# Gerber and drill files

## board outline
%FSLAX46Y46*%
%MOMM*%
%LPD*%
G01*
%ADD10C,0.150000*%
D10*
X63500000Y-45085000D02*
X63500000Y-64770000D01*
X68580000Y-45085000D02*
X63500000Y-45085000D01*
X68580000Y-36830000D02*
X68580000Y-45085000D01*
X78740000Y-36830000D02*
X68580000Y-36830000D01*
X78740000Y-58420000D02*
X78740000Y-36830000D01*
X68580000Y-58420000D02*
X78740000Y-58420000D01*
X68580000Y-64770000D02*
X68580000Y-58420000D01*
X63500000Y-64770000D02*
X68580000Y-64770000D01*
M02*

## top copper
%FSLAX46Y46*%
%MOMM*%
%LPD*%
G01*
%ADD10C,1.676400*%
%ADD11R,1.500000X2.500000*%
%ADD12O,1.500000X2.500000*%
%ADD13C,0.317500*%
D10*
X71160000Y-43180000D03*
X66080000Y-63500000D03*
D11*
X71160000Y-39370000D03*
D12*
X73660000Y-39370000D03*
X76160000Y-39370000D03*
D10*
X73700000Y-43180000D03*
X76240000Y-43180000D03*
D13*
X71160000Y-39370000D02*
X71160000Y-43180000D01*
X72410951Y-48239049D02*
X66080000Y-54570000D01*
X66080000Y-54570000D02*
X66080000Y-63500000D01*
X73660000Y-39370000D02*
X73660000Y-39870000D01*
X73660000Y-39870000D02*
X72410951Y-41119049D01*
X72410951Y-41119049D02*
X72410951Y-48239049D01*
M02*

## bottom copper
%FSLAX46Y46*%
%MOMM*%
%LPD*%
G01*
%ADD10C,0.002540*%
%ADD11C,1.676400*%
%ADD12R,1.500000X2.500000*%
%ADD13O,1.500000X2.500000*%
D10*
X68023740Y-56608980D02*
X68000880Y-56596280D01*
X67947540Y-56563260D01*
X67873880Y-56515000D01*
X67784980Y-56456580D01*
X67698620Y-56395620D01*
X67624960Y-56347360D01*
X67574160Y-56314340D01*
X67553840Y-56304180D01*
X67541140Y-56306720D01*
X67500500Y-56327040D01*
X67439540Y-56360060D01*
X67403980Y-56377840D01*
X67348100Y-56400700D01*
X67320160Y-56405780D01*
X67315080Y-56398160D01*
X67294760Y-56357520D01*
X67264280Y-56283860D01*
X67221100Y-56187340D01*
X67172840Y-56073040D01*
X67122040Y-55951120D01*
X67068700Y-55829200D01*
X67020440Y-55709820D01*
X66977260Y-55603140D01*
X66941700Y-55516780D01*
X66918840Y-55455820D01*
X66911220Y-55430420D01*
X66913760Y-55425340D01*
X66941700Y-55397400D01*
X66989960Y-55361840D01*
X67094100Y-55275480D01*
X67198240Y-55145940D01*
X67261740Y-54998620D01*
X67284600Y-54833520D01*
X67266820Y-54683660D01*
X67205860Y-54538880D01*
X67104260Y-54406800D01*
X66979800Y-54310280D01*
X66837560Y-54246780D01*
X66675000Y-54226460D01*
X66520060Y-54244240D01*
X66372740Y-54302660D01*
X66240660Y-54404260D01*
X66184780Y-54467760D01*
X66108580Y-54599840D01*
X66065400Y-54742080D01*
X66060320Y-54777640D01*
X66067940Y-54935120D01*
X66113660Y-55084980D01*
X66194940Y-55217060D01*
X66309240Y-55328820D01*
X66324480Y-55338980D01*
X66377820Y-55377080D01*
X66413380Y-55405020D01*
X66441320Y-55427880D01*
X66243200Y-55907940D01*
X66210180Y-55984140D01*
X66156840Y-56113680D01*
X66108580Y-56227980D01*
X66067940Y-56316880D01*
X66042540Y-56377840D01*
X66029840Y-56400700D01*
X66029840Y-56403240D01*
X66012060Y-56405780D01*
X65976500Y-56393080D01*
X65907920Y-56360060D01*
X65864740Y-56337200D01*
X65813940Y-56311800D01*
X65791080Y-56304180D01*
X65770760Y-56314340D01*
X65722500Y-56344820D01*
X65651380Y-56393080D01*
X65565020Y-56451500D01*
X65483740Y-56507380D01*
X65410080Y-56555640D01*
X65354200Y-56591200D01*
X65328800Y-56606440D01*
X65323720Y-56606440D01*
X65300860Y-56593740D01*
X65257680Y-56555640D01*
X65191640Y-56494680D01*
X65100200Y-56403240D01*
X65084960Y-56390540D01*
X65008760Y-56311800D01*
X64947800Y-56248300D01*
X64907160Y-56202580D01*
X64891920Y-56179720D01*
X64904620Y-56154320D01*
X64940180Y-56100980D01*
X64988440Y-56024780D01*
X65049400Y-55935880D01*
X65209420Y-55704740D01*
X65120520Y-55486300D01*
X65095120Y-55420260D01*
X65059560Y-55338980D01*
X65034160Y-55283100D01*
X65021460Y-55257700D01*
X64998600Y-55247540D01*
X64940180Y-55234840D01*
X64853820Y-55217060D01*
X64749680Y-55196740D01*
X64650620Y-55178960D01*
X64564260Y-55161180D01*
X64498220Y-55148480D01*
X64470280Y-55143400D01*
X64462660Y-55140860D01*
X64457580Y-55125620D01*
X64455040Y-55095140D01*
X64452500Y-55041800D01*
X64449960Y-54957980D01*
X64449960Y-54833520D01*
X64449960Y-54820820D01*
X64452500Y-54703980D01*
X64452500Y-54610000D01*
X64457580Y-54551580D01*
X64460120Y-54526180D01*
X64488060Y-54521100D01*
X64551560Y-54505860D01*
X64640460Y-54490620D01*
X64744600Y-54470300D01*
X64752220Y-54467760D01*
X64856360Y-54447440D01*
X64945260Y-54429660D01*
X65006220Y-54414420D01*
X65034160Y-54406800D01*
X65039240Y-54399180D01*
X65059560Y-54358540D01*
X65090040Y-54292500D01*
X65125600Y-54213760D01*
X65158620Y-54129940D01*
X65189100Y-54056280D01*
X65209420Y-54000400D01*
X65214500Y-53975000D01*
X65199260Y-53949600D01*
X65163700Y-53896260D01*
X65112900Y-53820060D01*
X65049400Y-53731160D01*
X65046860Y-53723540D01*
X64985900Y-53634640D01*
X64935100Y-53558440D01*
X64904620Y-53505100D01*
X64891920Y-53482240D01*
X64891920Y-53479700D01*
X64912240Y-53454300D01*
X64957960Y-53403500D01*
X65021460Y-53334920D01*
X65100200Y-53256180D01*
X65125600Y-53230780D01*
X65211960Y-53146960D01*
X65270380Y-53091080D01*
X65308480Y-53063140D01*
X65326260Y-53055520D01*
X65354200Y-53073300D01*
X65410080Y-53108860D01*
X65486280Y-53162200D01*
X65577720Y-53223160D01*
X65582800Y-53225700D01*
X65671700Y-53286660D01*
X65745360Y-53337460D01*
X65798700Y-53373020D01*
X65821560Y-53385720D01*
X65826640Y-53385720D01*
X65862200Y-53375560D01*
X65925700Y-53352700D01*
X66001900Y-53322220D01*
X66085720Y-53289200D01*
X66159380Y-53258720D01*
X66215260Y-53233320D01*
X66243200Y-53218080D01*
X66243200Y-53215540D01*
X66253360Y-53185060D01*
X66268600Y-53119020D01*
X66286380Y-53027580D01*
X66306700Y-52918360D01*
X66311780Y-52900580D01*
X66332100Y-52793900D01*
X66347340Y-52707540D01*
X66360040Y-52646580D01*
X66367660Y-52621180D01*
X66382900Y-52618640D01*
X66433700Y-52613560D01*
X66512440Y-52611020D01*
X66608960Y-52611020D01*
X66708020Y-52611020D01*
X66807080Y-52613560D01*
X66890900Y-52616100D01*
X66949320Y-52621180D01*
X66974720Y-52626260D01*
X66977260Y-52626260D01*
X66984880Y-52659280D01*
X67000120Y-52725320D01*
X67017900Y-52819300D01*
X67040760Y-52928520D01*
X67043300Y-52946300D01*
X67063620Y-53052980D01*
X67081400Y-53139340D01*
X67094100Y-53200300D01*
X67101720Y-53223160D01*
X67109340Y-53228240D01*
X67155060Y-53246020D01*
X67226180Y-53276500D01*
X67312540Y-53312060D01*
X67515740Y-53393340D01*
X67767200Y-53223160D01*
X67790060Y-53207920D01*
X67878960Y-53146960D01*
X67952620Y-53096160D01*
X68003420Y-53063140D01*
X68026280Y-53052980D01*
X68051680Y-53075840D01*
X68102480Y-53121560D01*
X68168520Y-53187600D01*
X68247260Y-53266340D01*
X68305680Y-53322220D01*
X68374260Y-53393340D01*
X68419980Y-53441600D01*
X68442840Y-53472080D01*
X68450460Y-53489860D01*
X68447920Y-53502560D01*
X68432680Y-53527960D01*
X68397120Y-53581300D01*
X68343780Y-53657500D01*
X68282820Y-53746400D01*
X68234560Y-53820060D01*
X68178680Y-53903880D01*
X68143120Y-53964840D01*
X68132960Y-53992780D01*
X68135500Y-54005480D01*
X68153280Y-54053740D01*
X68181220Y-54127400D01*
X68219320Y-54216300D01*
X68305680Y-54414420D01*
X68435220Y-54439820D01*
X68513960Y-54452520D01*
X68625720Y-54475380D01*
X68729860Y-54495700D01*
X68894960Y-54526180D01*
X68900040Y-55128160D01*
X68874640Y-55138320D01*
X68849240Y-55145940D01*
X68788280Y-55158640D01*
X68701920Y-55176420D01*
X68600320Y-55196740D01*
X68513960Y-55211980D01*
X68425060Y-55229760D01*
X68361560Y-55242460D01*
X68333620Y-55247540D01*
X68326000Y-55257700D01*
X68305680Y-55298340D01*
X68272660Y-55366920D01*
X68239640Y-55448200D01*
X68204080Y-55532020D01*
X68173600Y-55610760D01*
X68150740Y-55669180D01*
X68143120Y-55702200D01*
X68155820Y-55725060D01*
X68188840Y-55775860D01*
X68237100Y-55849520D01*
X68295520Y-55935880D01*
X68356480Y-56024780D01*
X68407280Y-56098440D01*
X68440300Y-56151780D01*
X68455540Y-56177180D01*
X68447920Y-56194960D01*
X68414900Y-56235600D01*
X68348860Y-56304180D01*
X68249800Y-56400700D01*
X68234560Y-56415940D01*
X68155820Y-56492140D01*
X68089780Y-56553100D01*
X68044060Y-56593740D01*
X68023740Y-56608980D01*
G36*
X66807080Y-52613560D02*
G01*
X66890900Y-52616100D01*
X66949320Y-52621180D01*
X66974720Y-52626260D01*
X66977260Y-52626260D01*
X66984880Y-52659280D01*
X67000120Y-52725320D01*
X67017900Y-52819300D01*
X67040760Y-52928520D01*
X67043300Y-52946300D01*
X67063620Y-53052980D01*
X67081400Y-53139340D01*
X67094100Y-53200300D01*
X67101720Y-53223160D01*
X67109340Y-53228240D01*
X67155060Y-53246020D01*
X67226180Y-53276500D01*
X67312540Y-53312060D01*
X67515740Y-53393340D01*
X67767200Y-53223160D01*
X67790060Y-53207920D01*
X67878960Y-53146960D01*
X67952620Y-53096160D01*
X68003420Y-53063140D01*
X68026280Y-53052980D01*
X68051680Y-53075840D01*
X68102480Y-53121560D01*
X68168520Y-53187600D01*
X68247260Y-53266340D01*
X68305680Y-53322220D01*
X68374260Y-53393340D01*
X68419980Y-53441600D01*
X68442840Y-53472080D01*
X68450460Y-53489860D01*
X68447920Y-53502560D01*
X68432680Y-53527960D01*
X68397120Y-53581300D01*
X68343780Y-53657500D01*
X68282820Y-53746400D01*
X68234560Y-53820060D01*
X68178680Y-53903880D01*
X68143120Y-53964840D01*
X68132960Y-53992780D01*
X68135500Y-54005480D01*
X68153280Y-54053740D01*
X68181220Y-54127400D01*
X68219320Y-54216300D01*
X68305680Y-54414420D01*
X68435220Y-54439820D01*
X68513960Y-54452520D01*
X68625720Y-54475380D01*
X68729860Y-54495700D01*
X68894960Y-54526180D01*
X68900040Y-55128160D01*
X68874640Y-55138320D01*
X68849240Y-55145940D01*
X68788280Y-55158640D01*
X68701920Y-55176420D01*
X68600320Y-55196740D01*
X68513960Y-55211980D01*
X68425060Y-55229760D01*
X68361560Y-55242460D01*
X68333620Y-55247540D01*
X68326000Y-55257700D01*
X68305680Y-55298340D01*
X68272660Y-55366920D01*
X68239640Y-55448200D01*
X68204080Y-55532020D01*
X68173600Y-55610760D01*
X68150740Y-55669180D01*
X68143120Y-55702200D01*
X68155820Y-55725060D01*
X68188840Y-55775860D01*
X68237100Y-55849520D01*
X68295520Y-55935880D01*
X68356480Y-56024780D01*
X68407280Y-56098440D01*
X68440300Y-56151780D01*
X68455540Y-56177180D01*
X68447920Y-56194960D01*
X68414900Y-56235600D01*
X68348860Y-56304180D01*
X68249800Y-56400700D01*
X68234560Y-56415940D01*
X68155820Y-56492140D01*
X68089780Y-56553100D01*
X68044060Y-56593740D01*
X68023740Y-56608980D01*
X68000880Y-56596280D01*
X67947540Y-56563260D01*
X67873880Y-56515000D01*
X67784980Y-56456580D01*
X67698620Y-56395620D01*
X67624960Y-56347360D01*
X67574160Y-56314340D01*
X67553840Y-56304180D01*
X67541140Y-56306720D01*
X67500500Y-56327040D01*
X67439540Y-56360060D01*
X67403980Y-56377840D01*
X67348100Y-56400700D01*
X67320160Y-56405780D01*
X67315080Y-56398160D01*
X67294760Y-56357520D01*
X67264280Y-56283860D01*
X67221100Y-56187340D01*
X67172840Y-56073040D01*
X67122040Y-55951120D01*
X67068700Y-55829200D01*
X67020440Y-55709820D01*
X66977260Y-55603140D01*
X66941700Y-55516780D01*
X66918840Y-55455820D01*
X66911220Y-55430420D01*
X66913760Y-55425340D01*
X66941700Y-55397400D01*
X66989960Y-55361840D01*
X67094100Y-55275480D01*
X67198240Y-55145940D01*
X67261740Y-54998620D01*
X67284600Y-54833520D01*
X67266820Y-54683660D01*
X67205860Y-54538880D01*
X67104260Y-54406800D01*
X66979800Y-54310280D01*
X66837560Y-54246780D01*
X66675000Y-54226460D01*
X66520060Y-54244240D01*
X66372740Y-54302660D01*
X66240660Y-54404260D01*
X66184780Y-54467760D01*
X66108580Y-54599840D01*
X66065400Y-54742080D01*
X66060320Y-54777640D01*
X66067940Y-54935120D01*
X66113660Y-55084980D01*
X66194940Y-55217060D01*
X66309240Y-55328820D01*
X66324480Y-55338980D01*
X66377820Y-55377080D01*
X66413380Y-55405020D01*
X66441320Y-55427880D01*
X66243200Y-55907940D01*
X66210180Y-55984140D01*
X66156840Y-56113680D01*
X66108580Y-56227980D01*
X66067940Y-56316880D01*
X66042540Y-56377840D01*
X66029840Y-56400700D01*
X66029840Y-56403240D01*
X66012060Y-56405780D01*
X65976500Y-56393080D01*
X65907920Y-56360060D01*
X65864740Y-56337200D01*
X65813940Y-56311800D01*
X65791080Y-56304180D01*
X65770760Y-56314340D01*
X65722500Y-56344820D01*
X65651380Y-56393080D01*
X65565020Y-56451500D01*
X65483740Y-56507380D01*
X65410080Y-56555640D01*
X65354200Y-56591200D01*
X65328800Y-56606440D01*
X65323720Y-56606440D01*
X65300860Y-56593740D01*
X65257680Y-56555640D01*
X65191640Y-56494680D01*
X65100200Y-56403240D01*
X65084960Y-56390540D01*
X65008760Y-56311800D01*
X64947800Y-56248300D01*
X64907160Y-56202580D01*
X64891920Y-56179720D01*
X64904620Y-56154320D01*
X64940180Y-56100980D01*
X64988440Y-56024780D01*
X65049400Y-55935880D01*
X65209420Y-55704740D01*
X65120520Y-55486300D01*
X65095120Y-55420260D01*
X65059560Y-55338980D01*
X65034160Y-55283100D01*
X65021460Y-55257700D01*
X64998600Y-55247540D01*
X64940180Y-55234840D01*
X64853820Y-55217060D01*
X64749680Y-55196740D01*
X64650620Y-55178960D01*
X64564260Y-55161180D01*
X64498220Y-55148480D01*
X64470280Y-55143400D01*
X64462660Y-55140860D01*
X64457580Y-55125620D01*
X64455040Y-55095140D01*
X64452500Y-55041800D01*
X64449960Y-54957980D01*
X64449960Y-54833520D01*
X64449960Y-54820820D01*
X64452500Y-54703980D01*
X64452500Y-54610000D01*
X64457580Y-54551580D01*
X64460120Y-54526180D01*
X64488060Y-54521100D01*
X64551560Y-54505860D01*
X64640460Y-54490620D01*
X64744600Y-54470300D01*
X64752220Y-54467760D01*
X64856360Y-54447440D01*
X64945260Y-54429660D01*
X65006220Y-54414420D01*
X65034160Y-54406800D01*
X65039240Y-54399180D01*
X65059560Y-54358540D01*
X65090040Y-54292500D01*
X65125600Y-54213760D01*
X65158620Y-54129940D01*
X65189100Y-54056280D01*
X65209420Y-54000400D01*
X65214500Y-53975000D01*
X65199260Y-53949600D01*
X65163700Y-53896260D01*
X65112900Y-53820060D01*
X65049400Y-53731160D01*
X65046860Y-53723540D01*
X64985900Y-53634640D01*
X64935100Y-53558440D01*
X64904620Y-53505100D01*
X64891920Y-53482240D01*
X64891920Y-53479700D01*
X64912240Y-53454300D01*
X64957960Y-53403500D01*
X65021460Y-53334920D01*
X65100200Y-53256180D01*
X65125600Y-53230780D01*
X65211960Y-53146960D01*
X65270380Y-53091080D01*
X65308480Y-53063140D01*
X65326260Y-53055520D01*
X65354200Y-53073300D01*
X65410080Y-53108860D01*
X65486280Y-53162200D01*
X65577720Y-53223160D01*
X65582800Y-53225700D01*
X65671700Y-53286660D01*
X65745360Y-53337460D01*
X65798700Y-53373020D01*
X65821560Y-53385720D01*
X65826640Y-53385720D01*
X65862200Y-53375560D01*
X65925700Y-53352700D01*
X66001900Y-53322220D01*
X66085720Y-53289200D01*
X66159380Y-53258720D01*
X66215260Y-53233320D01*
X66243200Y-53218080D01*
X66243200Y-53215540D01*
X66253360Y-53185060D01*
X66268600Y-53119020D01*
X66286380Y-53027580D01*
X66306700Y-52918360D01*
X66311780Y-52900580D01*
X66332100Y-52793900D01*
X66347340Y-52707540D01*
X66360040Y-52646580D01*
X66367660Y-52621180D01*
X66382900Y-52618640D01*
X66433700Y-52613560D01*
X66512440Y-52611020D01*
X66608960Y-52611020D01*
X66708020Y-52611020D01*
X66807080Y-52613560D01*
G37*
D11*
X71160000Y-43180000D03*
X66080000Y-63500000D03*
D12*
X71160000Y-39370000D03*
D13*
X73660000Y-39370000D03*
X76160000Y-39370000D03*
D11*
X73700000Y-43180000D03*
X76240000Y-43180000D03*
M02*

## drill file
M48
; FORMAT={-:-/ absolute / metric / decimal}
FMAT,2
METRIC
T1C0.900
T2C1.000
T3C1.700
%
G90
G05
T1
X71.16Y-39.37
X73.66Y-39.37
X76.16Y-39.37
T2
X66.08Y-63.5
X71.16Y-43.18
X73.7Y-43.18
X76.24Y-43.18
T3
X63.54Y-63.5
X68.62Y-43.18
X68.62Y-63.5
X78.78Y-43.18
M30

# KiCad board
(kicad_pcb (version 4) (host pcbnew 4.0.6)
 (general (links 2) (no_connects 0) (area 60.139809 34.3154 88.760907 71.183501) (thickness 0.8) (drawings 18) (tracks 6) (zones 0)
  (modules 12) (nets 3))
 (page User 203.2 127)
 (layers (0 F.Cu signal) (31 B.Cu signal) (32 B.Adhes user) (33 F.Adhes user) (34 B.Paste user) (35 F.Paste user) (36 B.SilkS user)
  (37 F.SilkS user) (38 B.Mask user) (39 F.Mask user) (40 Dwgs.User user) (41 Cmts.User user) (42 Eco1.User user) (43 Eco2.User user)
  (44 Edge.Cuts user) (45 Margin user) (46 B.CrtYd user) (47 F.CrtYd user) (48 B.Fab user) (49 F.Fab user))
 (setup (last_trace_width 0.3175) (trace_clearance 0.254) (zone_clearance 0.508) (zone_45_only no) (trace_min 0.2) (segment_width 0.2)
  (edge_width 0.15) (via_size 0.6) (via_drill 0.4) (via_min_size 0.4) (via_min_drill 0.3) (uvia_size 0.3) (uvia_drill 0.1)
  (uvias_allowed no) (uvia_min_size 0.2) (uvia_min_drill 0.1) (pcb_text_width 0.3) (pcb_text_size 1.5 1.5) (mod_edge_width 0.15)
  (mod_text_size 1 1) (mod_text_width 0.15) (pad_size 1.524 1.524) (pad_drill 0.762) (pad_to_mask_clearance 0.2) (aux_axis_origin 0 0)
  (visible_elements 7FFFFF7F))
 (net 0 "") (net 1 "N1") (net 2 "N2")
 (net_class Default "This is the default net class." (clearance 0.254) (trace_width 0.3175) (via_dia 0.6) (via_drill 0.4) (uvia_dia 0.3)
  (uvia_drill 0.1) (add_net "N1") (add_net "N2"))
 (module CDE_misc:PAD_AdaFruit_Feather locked (layer F.Cu) (at 71.12 43.18)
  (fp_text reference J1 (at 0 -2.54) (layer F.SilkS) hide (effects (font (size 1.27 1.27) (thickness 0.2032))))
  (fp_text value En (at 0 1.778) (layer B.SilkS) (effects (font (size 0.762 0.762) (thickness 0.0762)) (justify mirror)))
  (pad 1 thru_hole circle (at 0.04 0) (size 1.6764 1.6764) (drill 1) (layers *.Cu *.Mask) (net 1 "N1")))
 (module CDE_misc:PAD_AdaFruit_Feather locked (layer F.Cu) (at 66.04 63.5)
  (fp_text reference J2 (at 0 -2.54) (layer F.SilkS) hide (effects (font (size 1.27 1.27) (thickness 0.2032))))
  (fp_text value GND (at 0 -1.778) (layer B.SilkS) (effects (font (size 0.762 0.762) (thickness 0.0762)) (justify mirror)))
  (pad 1 thru_hole circle (at 0.04 0) (size 1.6764 1.6764) (drill 1) (layers *.Cu *.Mask) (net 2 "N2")))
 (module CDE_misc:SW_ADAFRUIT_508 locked (layer F.Cu) (at 71.12 39.37)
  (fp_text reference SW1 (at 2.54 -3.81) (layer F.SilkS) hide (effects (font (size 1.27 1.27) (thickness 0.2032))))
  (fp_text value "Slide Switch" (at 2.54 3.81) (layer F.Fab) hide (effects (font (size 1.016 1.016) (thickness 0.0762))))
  (pad 1 thru_hole rect (at 0.04 0) (size 1.5 2.5) (drill 0.9) (layers *.Cu *.Mask) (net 1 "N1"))
  (pad 2 thru_hole oval (at 2.54 0) (size 1.5 2.5) (drill 0.9) (layers *.Cu *.Mask) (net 2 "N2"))
  (pad 3 thru_hole oval (at 5.04 0) (size 1.5 2.5) (drill 0.9) (layers *.Cu *.Mask)))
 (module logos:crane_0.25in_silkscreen (layer B.Cu) (at 73.66 53.975 180)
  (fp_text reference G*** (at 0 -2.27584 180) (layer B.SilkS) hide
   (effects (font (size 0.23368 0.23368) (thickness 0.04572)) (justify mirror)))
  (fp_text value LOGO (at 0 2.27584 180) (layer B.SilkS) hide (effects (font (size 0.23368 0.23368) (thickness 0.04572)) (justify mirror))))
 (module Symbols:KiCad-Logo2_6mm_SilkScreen (layer F.Cu) (at 71.12 54.61)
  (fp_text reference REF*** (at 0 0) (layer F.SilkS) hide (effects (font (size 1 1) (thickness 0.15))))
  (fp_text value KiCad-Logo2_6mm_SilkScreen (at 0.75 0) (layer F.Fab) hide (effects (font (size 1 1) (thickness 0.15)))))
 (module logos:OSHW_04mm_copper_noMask (layer B.Cu) (at 66.675 54.61 180)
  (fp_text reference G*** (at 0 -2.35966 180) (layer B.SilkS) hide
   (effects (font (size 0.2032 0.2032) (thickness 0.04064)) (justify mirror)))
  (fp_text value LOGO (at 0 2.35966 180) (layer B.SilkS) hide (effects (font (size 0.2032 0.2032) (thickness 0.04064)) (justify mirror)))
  (fp_poly
   (pts (xy -1.34874 -1.99898) (xy -1.32588 -1.98628) (xy -1.27254 -1.95326) (xy -1.19888 -1.905) (xy -1.10998 -1.84658)
    (xy -1.02362 -1.78562) (xy -0.94996 -1.73736) (xy -0.89916 -1.70434) (xy -0.87884 -1.69418) (xy -0.86614 -1.69672) (xy -0.8255 -1.71704)
    (xy -0.76454 -1.75006) (xy -0.72898 -1.76784) (xy -0.6731 -1.7907) (xy -0.64516 -1.79578) (xy -0.64008 -1.78816) (xy -0.61976 -1.74752)
    (xy -0.58928 -1.67386) (xy -0.5461 -1.57734) (xy -0.49784 -1.46304) (xy -0.44704 -1.34112) (xy -0.3937 -1.2192) (xy -0.34544 -1.09982)
    (xy -0.30226 -0.99314) (xy -0.2667 -0.90678) (xy -0.24384 -0.84582) (xy -0.23622 -0.82042) (xy -0.23876 -0.81534) (xy -0.2667 -0.7874)
    (xy -0.31496 -0.75184) (xy -0.4191 -0.66548) (xy -0.52324 -0.53594) (xy -0.58674 -0.38862) (xy -0.6096 -0.22352) (xy -0.59182 -0.07366)
    (xy -0.53086 0.07112) (xy -0.42926 0.2032) (xy -0.3048 0.29972) (xy -0.16256 0.36322) (xy 0 0.38354) (xy 0.15494 0.36576)
    (xy 0.30226 0.30734) (xy 0.43434 0.20574) (xy 0.49022 0.14224) (xy 0.56642 0.01016) (xy 0.6096 -0.13208) (xy 0.61468 -0.16764)
    (xy 0.60706 -0.32512) (xy 0.56134 -0.47498) (xy 0.48006 -0.60706) (xy 0.36576 -0.71882) (xy 0.35052 -0.72898) (xy 0.29718 -0.76708)
    (xy 0.26162 -0.79502) (xy 0.23368 -0.81788) (xy 0.4318 -1.29794) (xy 0.46482 -1.37414) (xy 0.51816 -1.50368) (xy 0.56642 -1.61798)
    (xy 0.60706 -1.70688) (xy 0.63246 -1.76784) (xy 0.64516 -1.7907) (xy 0.64516 -1.79324) (xy 0.66294 -1.79578) (xy 0.6985 -1.78308)
    (xy 0.76708 -1.75006) (xy 0.81026 -1.7272) (xy 0.86106 -1.7018) (xy 0.88392 -1.69418) (xy 0.90424 -1.70434) (xy 0.9525 -1.73482)
    (xy 1.02362 -1.78308) (xy 1.10998 -1.8415) (xy 1.19126 -1.89738) (xy 1.26492 -1.94564) (xy 1.3208 -1.9812) (xy 1.3462 -1.99644)
    (xy 1.35128 -1.99644) (xy 1.37414 -1.98374) (xy 1.41732 -1.94564) (xy 1.48336 -1.88468) (xy 1.5748 -1.79324) (xy 1.59004 -1.78054)
    (xy 1.66624 -1.7018) (xy 1.7272 -1.6383) (xy 1.76784 -1.59258) (xy 1.78308 -1.56972) (xy 1.78308 -1.56972) (xy 1.77038 -1.54432)
    (xy 1.73482 -1.49098) (xy 1.68656 -1.41478) (xy 1.6256 -1.32588) (xy 1.46558 -1.09474) (xy 1.55448 -0.8763) (xy 1.57988 -0.81026)
    (xy 1.61544 -0.72898) (xy 1.64084 -0.6731) (xy 1.65354 -0.6477) (xy 1.6764 -0.63754) (xy 1.73482 -0.62484) (xy 1.82118 -0.60706)
    (xy 1.92532 -0.58674) (xy 2.02438 -0.56896) (xy 2.11074 -0.55118) (xy 2.17678 -0.53848) (xy 2.20472 -0.5334) (xy 2.21234 -0.53086)
    (xy 2.21742 -0.51562) (xy 2.21996 -0.48514) (xy 2.2225 -0.4318) (xy 2.22504 -0.34798) (xy 2.22504 -0.22352) (xy 2.22504 -0.21082)
    (xy 2.2225 -0.09398) (xy 2.2225 0) (xy 2.21742 0.05842) (xy 2.21488 0.08382) (xy 2.21488 0.08382) (xy 2.18694 0.0889)
    (xy 2.12344 0.10414) (xy 2.03454 0.11938) (xy 1.9304 0.1397) (xy 1.92278 0.14224) (xy 1.81864 0.16256) (xy 1.72974 0.18034)
    (xy 1.66878 0.19558) (xy 1.64084 0.2032) (xy 1.63576 0.21082) (xy 1.61544 0.25146) (xy 1.58496 0.3175) (xy 1.5494 0.39624)
    (xy 1.51638 0.48006) (xy 1.4859 0.55372) (xy 1.46558 0.6096) (xy 1.4605 0.635) (xy 1.4605 0.635) (xy 1.47574 0.6604) (xy 1.5113 0.71374)
    (xy 1.5621 0.78994) (xy 1.6256 0.87884) (xy 1.62814 0.88646) (xy 1.6891 0.97536) (xy 1.7399 1.05156) (xy 1.77038 1.1049)
    (xy 1.78308 1.12776) (xy 1.78308 1.1303) (xy 1.76276 1.1557) (xy 1.71704 1.2065) (xy 1.65354 1.27508) (xy 1.5748 1.35382)
    (xy 1.5494 1.37922) (xy 1.46304 1.46304) (xy 1.40462 1.51892) (xy 1.36652 1.54686) (xy 1.34874 1.55448) (xy 1.34874 1.55448)
    (xy 1.3208 1.5367) (xy 1.26492 1.50114) (xy 1.18872 1.4478) (xy 1.09728 1.38684) (xy 1.0922 1.3843) (xy 1.0033 1.32334)
    (xy 0.92964 1.27254) (xy 0.8763 1.23698) (xy 0.85344 1.22428) (xy 0.84836 1.22428) (xy 0.8128 1.23444) (xy 0.7493 1.2573)
    (xy 0.6731 1.28778) (xy 0.58928 1.3208) (xy 0.51562 1.35128) (xy 0.45974 1.37668) (xy 0.4318 1.39192) (xy 0.4318 1.39446)
    (xy 0.42164 1.42494) (xy 0.4064 1.49098) (xy 0.38862 1.58242) (xy 0.3683 1.69164) (xy 0.36322 1.70942) (xy 0.3429 1.8161)
    (xy 0.32766 1.90246) (xy 0.31496 1.96342) (xy 0.30734 1.98882) (xy 0.2921 1.99136) (xy 0.2413 1.99644) (xy 0.16256 1.99898)
    (xy 0.06604 1.99898) (xy -0.03302 1.99898) (xy -0.13208 1.99644) (xy -0.2159 1.9939) (xy -0.27432 1.98882) (xy -0.29972 1.98374)
    (xy -0.30226 1.98374) (xy -0.30988 1.95072) (xy -0.32512 1.88468) (xy -0.3429 1.7907) (xy -0.36576 1.68148) (xy -0.3683 1.6637)
    (xy -0.38862 1.55702) (xy -0.4064 1.47066) (xy -0.4191 1.4097) (xy -0.42672 1.38684) (xy -0.43434 1.38176) (xy -0.48006 1.36398)
    (xy -0.55118 1.3335) (xy -0.63754 1.29794) (xy -0.84074 1.21666) (xy -1.0922 1.38684) (xy -1.11506 1.40208) (xy -1.20396 1.46304)
    (xy -1.27762 1.51384) (xy -1.32842 1.54686) (xy -1.35128 1.55702) (xy -1.35128 1.55702) (xy -1.37668 1.53416) (xy -1.42748 1.48844)
    (xy -1.49352 1.4224) (xy -1.57226 1.34366) (xy -1.63068 1.28778) (xy -1.69926 1.21666) (xy -1.74498 1.1684) (xy -1.76784 1.13792)
    (xy -1.77546 1.12014) (xy -1.77292 1.10744) (xy -1.75768 1.08204) (xy -1.72212 1.0287) (xy -1.66878 0.9525) (xy -1.60782 0.8636)
    (xy -1.55956 0.78994) (xy -1.50368 0.70612) (xy -1.46812 0.64516) (xy -1.45796 0.61722) (xy -1.4605 0.60452) (xy -1.47828 0.55626)
    (xy -1.50622 0.4826) (xy -1.54432 0.3937) (xy -1.63068 0.19558) (xy -1.76022 0.17018) (xy -1.83896 0.15748) (xy -1.95072 0.13462)
    (xy -2.05486 0.1143) (xy -2.21996 0.08382) (xy -2.22504 -0.51816) (xy -2.19964 -0.52832) (xy -2.17424 -0.53594) (xy -2.11328 -0.54864)
    (xy -2.02692 -0.56642) (xy -1.92532 -0.58674) (xy -1.83896 -0.60198) (xy -1.75006 -0.61976) (xy -1.68656 -0.63246)
    (xy -1.65862 -0.63754) (xy -1.651 -0.6477) (xy -1.63068 -0.68834) (xy -1.59766 -0.75692) (xy -1.56464 -0.8382) (xy -1.52908 -0.92202)
    (xy -1.4986 -1.00076) (xy -1.47574 -1.05918) (xy -1.46812 -1.0922) (xy -1.48082 -1.11506) (xy -1.51384 -1.16586) (xy -1.5621 -1.23952)
    (xy -1.62052 -1.32588) (xy -1.68148 -1.41478) (xy -1.73228 -1.48844) (xy -1.7653 -1.54178) (xy -1.78054 -1.56718) (xy -1.77292 -1.58496)
    (xy -1.7399 -1.6256) (xy -1.67386 -1.69418) (xy -1.5748 -1.7907) (xy -1.55956 -1.80594) (xy -1.48082 -1.88214) (xy -1.41478 -1.9431)
    (xy -1.36906 -1.98374) (xy -1.34874 -1.99898))
   (layer B.Cu) (width 0.00254)))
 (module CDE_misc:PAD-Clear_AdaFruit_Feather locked (layer F.Cu) (at 68.58 63.5)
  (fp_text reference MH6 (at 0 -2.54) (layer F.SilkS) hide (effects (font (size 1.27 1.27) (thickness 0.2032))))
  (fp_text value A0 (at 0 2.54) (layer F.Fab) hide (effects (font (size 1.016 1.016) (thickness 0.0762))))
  (pad "" np_thru_hole circle (at 0.04 0) (size 1.7 1.7) (drill 1.7) (layers *.Cu *.Mask) (solder_mask_margin 0.001) (zone_connect 0)))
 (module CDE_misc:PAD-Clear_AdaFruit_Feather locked (layer F.Cu) (at 63.5 63.5)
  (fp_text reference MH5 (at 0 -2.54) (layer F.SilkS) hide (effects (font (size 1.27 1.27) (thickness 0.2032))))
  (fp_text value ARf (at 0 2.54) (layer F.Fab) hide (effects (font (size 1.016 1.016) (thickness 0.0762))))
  (pad "" np_thru_hole circle (at 0.04 0) (size 1.7 1.7) (drill 1.7) (layers *.Cu *.Mask) (solder_mask_margin 0.001) (zone_connect 0)))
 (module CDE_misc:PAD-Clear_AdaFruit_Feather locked (layer F.Cu) (at 78.74 43.18)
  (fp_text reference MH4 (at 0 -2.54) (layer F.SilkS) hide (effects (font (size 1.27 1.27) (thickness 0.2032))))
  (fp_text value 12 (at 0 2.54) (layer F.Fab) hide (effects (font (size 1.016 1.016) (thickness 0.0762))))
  (pad "" np_thru_hole circle (at 0.04 0) (size 1.7 1.7) (drill 1.7) (layers *.Cu *.Mask) (solder_mask_margin 0.001) (zone_connect 0)))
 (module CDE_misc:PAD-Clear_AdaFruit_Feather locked (layer F.Cu) (at 68.58 43.18)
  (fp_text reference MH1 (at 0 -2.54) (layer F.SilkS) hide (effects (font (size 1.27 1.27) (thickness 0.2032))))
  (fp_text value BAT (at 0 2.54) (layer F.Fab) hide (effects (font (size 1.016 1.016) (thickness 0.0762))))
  (pad "" np_thru_hole circle (at 0.04 0) (size 1.7 1.7) (drill 1.7) (layers *.Cu *.Mask) (solder_mask_margin 0.001) (zone_connect 0)))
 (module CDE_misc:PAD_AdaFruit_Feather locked (layer F.Cu) (at 73.66 43.18)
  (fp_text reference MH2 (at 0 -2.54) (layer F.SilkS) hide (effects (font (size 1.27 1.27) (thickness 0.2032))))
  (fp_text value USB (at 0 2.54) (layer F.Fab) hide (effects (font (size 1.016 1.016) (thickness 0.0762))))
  (pad 1 thru_hole circle (at 0.04 0) (size 1.6764 1.6764) (drill 1) (layers *.Cu *.Mask)))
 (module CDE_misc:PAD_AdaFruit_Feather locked (layer F.Cu) (at 76.2 43.18)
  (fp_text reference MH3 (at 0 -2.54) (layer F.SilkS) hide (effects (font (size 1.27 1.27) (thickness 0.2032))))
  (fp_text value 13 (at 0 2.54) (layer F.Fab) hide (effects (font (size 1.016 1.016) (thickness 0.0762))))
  (pad 1 thru_hole circle (at 0.04 0) (size 1.6764 1.6764) (drill 1) (layers *.Cu *.Mask)))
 (gr_line (start 63.5 45.085) (end 63.5 64.77) (angle 90) (layer Edge.Cuts) (width 0.15))
 (gr_line (start 68.58 45.085) (end 63.5 45.085) (angle 90) (layer Edge.Cuts) (width 0.15))
 (gr_line (start 68.58 36.83) (end 68.58 45.085) (angle 90) (layer Edge.Cuts) (width 0.15))
 (gr_line (start 78.74 36.83) (end 68.58 36.83) (angle 90) (layer Edge.Cuts) (width 0.15))
 (gr_line (start 78.74 58.42) (end 78.74 36.83) (angle 90) (layer Edge.Cuts) (width 0.15))
 (gr_line (start 68.58 58.42) (end 78.74 58.42) (angle 90) (layer Edge.Cuts) (width 0.15))
 (gr_line (start 68.58 64.77) (end 68.58 58.42) (angle 90) (layer Edge.Cuts) (width 0.15))
 (gr_line (start 63.5 64.77) (end 68.58 64.77) (angle 90) (layer Edge.Cuts) (width 0.15))
 (segment (start 71.16 39.37) (end 71.16 43.18) (width 0.3175) (layer F.Cu) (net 1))
 (segment (start 72.410951 48.239049) (end 66.08 54.57) (width 0.3175) (layer F.Cu) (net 2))
 (segment (start 66.08 54.57) (end 66.08 63.5) (width 0.3175) (layer F.Cu) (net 2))
 (segment (start 73.66 39.37) (end 73.66 39.87) (width 0.3175) (layer F.Cu) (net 2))
 (segment (start 73.66 39.87) (end 72.410951 41.119049) (width 0.3175) (layer F.Cu) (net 2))
 (segment (start 72.410951 41.119049) (end 72.410951 48.239049) (width 0.3175) (layer F.Cu) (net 2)))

